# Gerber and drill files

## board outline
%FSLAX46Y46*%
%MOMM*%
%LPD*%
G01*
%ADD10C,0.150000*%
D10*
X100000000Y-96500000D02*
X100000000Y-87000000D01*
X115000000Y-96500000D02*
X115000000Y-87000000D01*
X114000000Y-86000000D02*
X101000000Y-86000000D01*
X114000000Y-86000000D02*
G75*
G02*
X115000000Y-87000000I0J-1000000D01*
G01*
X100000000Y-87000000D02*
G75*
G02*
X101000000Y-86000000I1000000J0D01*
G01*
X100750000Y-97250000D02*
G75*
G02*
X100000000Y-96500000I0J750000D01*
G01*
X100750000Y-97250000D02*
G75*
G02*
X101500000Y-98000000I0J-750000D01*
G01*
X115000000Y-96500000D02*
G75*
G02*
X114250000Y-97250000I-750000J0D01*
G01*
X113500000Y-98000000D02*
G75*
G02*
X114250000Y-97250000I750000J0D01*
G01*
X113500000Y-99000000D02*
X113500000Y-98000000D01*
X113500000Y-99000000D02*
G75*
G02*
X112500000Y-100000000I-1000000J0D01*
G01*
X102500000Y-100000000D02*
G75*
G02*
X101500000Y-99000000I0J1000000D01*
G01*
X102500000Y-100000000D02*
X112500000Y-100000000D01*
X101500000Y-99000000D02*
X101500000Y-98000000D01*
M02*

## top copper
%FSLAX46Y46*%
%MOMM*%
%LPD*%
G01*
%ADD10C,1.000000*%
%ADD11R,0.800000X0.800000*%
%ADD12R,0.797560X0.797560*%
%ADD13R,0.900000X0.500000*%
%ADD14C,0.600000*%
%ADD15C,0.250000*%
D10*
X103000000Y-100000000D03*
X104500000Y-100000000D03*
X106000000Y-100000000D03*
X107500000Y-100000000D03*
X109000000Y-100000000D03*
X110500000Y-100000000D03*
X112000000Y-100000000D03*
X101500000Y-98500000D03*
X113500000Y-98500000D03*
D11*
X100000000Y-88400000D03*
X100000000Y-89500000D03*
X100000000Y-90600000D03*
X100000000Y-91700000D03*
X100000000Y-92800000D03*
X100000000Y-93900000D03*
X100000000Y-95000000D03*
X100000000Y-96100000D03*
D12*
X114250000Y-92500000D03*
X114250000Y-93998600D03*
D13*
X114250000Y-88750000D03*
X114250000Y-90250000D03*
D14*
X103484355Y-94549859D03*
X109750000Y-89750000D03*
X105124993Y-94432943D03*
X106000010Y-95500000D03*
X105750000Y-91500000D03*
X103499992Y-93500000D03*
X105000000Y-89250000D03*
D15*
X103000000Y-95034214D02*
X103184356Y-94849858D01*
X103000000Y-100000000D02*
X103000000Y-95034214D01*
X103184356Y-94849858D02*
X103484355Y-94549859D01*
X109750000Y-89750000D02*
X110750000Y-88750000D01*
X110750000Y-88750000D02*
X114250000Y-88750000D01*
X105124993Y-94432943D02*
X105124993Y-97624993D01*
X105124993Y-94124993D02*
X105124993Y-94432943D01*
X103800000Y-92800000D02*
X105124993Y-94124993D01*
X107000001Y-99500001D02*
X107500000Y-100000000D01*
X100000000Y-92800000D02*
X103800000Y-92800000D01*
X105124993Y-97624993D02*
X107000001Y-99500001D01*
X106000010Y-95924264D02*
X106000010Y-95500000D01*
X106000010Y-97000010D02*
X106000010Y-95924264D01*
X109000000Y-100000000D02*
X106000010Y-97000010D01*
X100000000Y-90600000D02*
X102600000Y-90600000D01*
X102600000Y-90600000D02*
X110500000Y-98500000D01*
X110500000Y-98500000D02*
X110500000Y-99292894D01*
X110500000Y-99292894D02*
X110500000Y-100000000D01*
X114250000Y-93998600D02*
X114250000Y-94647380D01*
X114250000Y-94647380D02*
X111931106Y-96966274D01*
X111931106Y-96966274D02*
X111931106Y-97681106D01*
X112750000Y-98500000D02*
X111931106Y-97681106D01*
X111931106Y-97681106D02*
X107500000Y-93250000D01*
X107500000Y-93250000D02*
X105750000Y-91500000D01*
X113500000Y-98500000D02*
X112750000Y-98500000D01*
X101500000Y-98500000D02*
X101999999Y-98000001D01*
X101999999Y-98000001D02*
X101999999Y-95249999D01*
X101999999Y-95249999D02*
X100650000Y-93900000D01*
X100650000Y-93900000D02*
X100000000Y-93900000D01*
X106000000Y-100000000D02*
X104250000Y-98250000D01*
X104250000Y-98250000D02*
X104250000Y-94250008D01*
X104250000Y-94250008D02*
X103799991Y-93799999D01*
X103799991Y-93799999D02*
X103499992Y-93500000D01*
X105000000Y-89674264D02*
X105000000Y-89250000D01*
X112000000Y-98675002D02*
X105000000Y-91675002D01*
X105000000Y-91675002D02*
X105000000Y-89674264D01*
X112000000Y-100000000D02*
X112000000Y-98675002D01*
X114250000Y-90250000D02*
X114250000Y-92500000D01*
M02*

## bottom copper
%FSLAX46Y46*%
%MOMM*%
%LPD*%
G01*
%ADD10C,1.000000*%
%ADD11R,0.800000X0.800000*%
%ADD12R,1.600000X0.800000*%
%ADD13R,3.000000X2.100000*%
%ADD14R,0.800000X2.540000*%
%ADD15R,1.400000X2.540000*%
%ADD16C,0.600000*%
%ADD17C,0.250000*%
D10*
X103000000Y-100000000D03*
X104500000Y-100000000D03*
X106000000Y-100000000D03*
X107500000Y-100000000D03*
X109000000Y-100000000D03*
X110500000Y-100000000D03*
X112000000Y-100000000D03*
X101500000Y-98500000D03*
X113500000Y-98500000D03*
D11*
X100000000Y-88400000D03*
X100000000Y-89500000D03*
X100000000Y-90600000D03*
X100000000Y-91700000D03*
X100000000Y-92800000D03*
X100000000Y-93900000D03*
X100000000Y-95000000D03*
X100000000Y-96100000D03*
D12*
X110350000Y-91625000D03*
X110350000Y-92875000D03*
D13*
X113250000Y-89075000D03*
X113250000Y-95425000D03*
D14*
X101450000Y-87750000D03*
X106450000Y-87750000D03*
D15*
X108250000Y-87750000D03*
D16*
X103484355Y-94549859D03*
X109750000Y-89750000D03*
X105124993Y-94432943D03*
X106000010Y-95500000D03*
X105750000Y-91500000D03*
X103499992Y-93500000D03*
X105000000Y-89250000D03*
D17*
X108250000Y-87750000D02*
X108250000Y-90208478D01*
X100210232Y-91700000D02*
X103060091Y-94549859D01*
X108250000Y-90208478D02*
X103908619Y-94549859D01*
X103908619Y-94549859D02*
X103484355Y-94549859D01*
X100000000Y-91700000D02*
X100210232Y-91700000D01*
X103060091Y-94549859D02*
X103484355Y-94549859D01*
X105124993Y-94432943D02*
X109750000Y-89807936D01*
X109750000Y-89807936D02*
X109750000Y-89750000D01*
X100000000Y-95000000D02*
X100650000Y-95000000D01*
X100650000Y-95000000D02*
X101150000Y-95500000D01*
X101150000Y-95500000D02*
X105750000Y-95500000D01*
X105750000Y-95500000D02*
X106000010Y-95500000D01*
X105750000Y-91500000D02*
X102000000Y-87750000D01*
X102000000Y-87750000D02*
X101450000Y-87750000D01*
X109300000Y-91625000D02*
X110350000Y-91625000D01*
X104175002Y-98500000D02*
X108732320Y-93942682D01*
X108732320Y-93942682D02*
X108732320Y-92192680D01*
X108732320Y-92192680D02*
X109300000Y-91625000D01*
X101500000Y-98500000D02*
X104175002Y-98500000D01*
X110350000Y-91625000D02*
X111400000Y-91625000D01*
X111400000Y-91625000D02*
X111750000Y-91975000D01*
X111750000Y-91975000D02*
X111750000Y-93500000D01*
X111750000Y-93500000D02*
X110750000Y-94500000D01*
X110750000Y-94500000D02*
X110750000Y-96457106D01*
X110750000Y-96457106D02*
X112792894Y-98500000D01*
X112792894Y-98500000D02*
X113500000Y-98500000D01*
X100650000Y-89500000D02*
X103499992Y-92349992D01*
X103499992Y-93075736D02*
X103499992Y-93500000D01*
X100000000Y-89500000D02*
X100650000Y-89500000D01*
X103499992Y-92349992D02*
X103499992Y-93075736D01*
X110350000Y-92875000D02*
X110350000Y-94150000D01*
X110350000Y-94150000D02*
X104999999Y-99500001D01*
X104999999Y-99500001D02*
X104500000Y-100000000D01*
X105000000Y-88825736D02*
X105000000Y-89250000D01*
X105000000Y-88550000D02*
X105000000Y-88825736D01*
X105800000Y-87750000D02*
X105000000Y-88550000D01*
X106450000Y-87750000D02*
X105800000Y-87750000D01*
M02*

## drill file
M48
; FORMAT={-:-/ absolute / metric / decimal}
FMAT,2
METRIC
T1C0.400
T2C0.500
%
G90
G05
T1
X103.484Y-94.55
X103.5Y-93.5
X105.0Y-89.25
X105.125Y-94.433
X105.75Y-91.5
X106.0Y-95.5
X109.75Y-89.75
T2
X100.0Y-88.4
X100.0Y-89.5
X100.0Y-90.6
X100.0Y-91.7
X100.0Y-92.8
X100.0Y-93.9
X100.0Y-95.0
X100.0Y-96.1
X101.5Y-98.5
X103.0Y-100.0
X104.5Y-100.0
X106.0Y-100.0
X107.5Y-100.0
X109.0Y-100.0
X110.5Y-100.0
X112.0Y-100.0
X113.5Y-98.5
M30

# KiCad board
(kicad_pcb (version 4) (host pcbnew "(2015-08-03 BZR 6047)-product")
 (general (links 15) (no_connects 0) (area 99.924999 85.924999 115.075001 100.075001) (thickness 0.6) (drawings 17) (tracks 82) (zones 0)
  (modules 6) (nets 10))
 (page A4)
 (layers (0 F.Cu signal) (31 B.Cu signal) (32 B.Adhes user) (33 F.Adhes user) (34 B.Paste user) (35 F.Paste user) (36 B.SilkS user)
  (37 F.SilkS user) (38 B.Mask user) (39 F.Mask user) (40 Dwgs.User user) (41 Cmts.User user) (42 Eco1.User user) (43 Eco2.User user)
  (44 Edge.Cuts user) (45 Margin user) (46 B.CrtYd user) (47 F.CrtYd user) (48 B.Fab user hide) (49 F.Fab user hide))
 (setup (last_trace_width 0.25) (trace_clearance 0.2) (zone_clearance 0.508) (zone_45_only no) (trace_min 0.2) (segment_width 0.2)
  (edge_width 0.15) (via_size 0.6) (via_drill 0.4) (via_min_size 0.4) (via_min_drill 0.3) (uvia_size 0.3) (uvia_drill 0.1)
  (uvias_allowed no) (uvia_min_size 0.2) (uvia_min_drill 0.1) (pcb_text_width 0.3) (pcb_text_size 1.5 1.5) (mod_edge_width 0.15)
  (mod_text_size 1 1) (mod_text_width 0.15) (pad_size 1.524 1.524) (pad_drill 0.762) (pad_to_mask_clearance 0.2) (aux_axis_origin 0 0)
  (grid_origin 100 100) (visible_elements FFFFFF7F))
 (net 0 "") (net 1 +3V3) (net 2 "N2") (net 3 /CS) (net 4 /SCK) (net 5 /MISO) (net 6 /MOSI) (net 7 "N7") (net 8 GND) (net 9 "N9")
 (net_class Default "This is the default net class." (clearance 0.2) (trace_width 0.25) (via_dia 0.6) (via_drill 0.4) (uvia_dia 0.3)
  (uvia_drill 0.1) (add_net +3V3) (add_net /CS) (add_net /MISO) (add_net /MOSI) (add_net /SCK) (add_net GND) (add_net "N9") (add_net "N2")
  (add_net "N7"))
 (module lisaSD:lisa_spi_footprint (layer F.Cu) (at 100 100)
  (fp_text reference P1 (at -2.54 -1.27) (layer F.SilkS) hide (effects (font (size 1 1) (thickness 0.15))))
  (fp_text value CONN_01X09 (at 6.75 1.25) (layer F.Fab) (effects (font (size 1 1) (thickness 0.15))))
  (pad 2 thru_hole circle (at 3 0) (size 1 1) (drill 0.5) (layers *.Cu *.Mask F.SilkS) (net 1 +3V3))
  (pad 3 thru_hole circle (at 4.5 0) (size 1 1) (drill 0.5) (layers *.Cu *.Mask F.SilkS) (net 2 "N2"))
  (pad 4 thru_hole circle (at 6 0) (size 1 1) (drill 0.5) (layers *.Cu *.Mask F.SilkS) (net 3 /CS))
  (pad 5 thru_hole circle (at 7.5 0) (size 1 1) (drill 0.5) (layers *.Cu *.Mask F.SilkS) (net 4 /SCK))
  (pad 6 thru_hole circle (at 9 0) (size 1 1) (drill 0.5) (layers *.Cu *.Mask F.SilkS) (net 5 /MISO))
  (pad 7 thru_hole circle (at 10.5 0) (size 1 1) (drill 0.5) (layers *.Cu *.Mask F.SilkS) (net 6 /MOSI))
  (pad 8 thru_hole circle (at 12 0) (size 1 1) (drill 0.5) (layers *.Cu *.Mask F.SilkS) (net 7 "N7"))
  (pad 1 thru_hole circle (at 1.5 -1.5) (size 1 1) (drill 0.5) (layers *.Cu *.Mask F.SilkS) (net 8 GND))
  (pad 9 thru_hole circle (at 13.5 -1.5) (size 1 1) (drill 0.5) (layers *.Cu *.Mask F.SilkS) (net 8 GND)))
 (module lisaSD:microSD (layer F.Cu) (at 100 97.1 90)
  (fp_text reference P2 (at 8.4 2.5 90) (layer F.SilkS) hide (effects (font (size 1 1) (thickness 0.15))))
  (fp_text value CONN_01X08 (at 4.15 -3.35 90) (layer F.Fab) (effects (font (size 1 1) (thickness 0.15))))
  (pad 1 thru_hole rect (at 8.7 0 90) (size 0.8 0.8) (drill 0.5) (layers *.Cu *.Mask F.SilkS))
  (pad 2 thru_hole rect (at 7.6 0 90) (size 0.8 0.8) (drill 0.5) (layers *.Cu *.Mask F.SilkS) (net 3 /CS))
  (pad 3 thru_hole rect (at 6.5 0 90) (size 0.8 0.8) (drill 0.5) (layers *.Cu *.Mask F.SilkS) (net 6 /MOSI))
  (pad 4 thru_hole rect (at 5.4 0 90) (size 0.8 0.8) (drill 0.5) (layers *.Cu *.Mask F.SilkS) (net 1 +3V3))
  (pad 5 thru_hole rect (at 4.3 0 90) (size 0.8 0.8) (drill 0.5) (layers *.Cu *.Mask F.SilkS) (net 4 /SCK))
  (pad 6 thru_hole rect (at 3.2 0 90) (size 0.8 0.8) (drill 0.5) (layers *.Cu *.Mask F.SilkS) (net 8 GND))
  (pad 7 thru_hole rect (at 2.1 0 90) (size 0.8 0.8) (drill 0.5) (layers *.Cu *.Mask F.SilkS) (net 5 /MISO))
  (pad 8 thru_hole rect (at 1 0 90) (size 0.8 0.8) (drill 0.5) (layers *.Cu *.Mask F.SilkS)))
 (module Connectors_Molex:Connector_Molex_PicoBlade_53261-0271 (layer B.Cu) (at 113.25 92.25 270)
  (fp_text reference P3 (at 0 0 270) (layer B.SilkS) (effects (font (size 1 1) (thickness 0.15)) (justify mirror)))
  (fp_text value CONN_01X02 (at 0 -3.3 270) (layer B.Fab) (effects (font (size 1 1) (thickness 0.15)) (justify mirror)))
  (pad 1 smd rect (at -0.625 2.9 270) (size 0.8 1.6) (layers B.Cu B.Paste B.Mask) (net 8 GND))
  (pad 2 smd rect (at 0.625 2.9 270) (size 0.8 1.6) (layers B.Cu B.Paste B.Mask) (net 2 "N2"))
  (pad "" smd rect (at -3.175 0 270) (size 2.1 3) (layers B.Cu B.Paste B.Mask))
  (pad "" smd rect (at 3.175 0 270) (size 2.1 3) (layers B.Cu B.Paste B.Mask)))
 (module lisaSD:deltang (layer B.Cu) (at 100.65 87.85)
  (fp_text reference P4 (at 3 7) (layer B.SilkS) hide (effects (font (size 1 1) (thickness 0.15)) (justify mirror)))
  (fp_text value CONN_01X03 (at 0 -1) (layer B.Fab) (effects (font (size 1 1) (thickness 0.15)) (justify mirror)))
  (pad 1 smd rect (at 0.8 -0.1) (size 0.8 2.54) (layers B.Cu B.Paste B.Mask) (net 8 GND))
  (pad 2 smd rect (at 5.8 -0.1) (size 0.8 2.54) (layers B.Cu B.Paste B.Mask) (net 7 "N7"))
  (pad 3 smd rect (at 7.6 -0.1) (size 1.4 2.54) (layers B.Cu B.Paste B.Mask) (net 1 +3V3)))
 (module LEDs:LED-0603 (layer F.Cu) (at 114.25 93.2493 90)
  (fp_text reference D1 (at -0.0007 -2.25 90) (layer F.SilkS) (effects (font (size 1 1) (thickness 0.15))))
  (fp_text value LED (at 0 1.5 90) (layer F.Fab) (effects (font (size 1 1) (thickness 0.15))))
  (pad 2 smd rect (at 0.7493 0 270) (size 0.79756 0.79756) (layers F.Cu F.Paste F.Mask) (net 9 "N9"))
  (pad 1 smd rect (at -0.7493 0 270) (size 0.79756 0.79756) (layers F.Cu F.Paste F.Mask) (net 8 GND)))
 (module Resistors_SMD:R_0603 (layer F.Cu) (at 114.25 89.5 270)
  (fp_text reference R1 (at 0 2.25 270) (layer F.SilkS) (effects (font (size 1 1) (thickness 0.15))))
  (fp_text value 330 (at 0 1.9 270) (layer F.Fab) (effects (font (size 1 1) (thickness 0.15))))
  (pad 1 smd rect (at -0.75 0 270) (size 0.5 0.9) (layers F.Cu F.Paste F.Mask) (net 4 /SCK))
  (pad 2 smd rect (at 0.75 0 270) (size 0.5 0.9) (layers F.Cu F.Paste F.Mask) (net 9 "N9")))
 (gr_line (start 100 96.5) (end 100 87) (layer Edge.Cuts) (width 0.15))
 (gr_line (start 115 96.5) (end 115 87) (layer Edge.Cuts) (width 0.15))
 (gr_line (start 114 86) (end 101 86) (angle 90) (layer Edge.Cuts) (width 0.15))
 (gr_arc (start 114 87) (end 114 86) (angle 90) (layer Edge.Cuts) (width 0.15))
 (gr_arc (start 101 87) (end 100 87) (angle 90) (layer Edge.Cuts) (width 0.15))
 (gr_arc (start 100.75 96.5) (end 100.75 97.25) (angle 90) (layer Edge.Cuts) (width 0.15))
 (gr_arc (start 100.75 98) (end 100.75 97.25) (angle 90) (layer Edge.Cuts) (width 0.15))
 (gr_arc (start 114.25 96.5) (end 115 96.5) (angle 90) (layer Edge.Cuts) (width 0.15))
 (gr_arc (start 114.25 98) (end 113.5 98) (angle 90) (layer Edge.Cuts) (width 0.15))
 (gr_line (start 113.5 99) (end 113.5 98) (angle 90) (layer Edge.Cuts) (width 0.15))
 (gr_arc (start 112.5 99) (end 113.5 99) (angle 90) (layer Edge.Cuts) (width 0.15))
 (gr_arc (start 102.5 99) (end 102.5 100) (angle 90) (layer Edge.Cuts) (width 0.15))
 (gr_line (start 102.5 100) (end 112.5 100) (angle 90) (layer Edge.Cuts) (width 0.15))
 (gr_line (start 101.5 99) (end 101.5 98) (angle 90) (layer Edge.Cuts) (width 0.15))
 (segment (start 103 95.034214) (end 103.184356 94.849858) (width 0.25) (layer F.Cu) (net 1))
 (segment (start 108.25 87.75) (end 108.25 90.208478) (width 0.25) (layer B.Cu) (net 1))
 (segment (start 100.210232 91.7) (end 103.060091 94.549859) (width 0.25) (layer B.Cu) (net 1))
 (segment (start 108.25 90.208478) (end 103.908619 94.549859) (width 0.25) (layer B.Cu) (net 1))
 (segment (start 103 100) (end 103 95.034214) (width 0.25) (layer F.Cu) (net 1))
 (segment (start 103.908619 94.549859) (end 103.484355 94.549859) (width 0.25) (layer B.Cu) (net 1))
 (via (at 103.484355 94.549859) (size 0.6) (drill 0.4) (layers F.Cu B.Cu) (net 1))
 (segment (start 100 91.7) (end 100.210232 91.7) (width 0.25) (layer B.Cu) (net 1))
 (segment (start 103.060091 94.549859) (end 103.484355 94.549859) (width 0.25) (layer B.Cu) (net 1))
 (segment (start 103.184356 94.849858) (end 103.484355 94.549859) (width 0.25) (layer F.Cu) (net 1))
 (segment (start 109.75 89.75) (end 110.75 88.75) (width 0.25) (layer F.Cu) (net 4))
 (segment (start 110.75 88.75) (end 114.25 88.75) (width 0.25) (layer F.Cu) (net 4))
 (segment (start 105.124993 94.432943) (end 109.75 89.807936) (width 0.25) (layer B.Cu) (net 4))
 (segment (start 109.75 89.807936) (end 109.75 89.75) (width 0.25) (layer B.Cu) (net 4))
 (via (at 109.75 89.75) (size 0.6) (drill 0.4) (layers F.Cu B.Cu) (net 4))
 (segment (start 105.124993 94.432943) (end 105.124993 97.624993) (width 0.25) (layer F.Cu) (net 4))
 (segment (start 105.124993 94.124993) (end 105.124993 94.432943) (width 0.25) (layer F.Cu) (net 4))
 (via (at 105.124993 94.432943) (size 0.6) (drill 0.4) (layers F.Cu B.Cu) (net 4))
 (segment (start 103.8 92.8) (end 105.124993 94.124993) (width 0.25) (layer F.Cu) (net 4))
 (segment (start 107.000001 99.500001) (end 107.5 100) (width 0.25) (layer F.Cu) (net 4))
 (segment (start 100 92.8) (end 103.8 92.8) (width 0.25) (layer F.Cu) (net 4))
 (segment (start 105.124993 97.624993) (end 107.000001 99.500001) (width 0.25) (layer F.Cu) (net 4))
 (segment (start 100 95) (end 100.65 95) (width 0.25) (layer B.Cu) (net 5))
 (segment (start 100.65 95) (end 101.15 95.5) (width 0.25) (layer B.Cu) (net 5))
 (segment (start 101.15 95.5) (end 105.75 95.5) (width 0.25) (layer B.Cu) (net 5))
 (segment (start 105.75 95.5) (end 106.00001 95.5) (width 0.25) (layer B.Cu) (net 5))
 (segment (start 106.00001 95.924264) (end 106.00001 95.5) (width 0.25) (layer F.Cu) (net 5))
 (segment (start 106.00001 97.00001) (end 106.00001 95.924264) (width 0.25) (layer F.Cu) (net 5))
 (via (at 106.00001 95.5) (size 0.6) (drill 0.4) (layers F.Cu B.Cu) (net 5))
 (segment (start 109 100) (end 106.00001 97.00001) (width 0.25) (layer F.Cu) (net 5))
 (segment (start 100 90.6) (end 102.6 90.6) (width 0.25) (layer F.Cu) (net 6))
 (segment (start 102.6 90.6) (end 110.5 98.5) (width 0.25) (layer F.Cu) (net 6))
 (segment (start 110.5 98.5) (end 110.5 99.292894) (width 0.25) (layer F.Cu) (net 6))
 (segment (start 110.5 99.292894) (end 110.5 100) (width 0.25) (layer F.Cu) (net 6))
 (segment (start 114.25 93.9986) (end 114.25 94.64738) (width 0.25) (layer F.Cu) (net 8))
 (segment (start 114.25 94.64738) (end 111.931106 96.966274) (width 0.25) (layer F.Cu) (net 8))
 (segment (start 111.931106 96.966274) (end 111.931106 97.681106) (width 0.25) (layer F.Cu) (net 8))
 (segment (start 112.75 98.5) (end 111.931106 97.681106) (width 0.25) (layer F.Cu) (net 8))
 (segment (start 111.931106 97.681106) (end 107.5 93.25) (width 0.25) (layer F.Cu) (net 8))
 (segment (start 105.75 91.5) (end 102 87.75) (width 0.25) (layer B.Cu) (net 8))
 (segment (start 102 87.75) (end 101.45 87.75) (width 0.25) (layer B.Cu) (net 8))
 (segment (start 107.5 93.25) (end 105.75 91.5) (width 0.25) (layer F.Cu) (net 8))
 (via (at 105.75 91.5) (size 0.6) (drill 0.4) (layers F.Cu B.Cu) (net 8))
 (segment (start 113.5 98.5) (end 112.75 98.5) (width 0.25) (layer F.Cu) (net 8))
 (segment (start 109.3 91.625) (end 110.35 91.625) (width 0.25) (layer B.Cu) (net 8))
 (segment (start 104.175002 98.5) (end 108.73232 93.942682) (width 0.25) (layer B.Cu) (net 8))
 (segment (start 108.73232 93.942682) (end 108.73232 92.19268) (width 0.25) (layer B.Cu) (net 8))
 (segment (start 108.73232 92.19268) (end 109.3 91.625) (width 0.25) (layer B.Cu) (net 8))
 (segment (start 101.5 98.5) (end 104.175002 98.5) (width 0.25) (layer B.Cu) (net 8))
 (segment (start 110.35 91.625) (end 111.4 91.625) (width 0.25) (layer B.Cu) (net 8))
 (segment (start 111.4 91.625) (end 111.75 91.975) (width 0.25) (layer B.Cu) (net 8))
 (segment (start 111.75 91.975) (end 111.75 93.5) (width 0.25) (layer B.Cu) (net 8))
 (segment (start 111.75 93.5) (end 110.75 94.5) (width 0.25) (layer B.Cu) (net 8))
 (segment (start 110.75 94.5) (end 110.75 96.457106) (width 0.25) (layer B.Cu) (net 8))
 (segment (start 110.75 96.457106) (end 112.792894 98.5) (width 0.25) (layer B.Cu) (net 8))
 (segment (start 112.792894 98.5) (end 113.5 98.5) (width 0.25) (layer B.Cu) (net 8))
 (segment (start 101.5 98.5) (end 101.999999 98.000001) (width 0.25) (layer F.Cu) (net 8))
 (segment (start 101.999999 98.000001) (end 101.999999 95.249999) (width 0.25) (layer F.Cu) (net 8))
 (segment (start 101.999999 95.249999) (end 100.65 93.9) (width 0.25) (layer F.Cu) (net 8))
 (segment (start 100.65 93.9) (end 100 93.9) (width 0.25) (layer F.Cu) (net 8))
 (segment (start 100.65 89.5) (end 103.499992 92.349992) (width 0.25) (layer B.Cu) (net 3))
 (segment (start 103.499992 93.075736) (end 103.499992 93.5) (width 0.25) (layer B.Cu) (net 3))
 (segment (start 106 100) (end 104.25 98.25) (width 0.25) (layer F.Cu) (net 3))
 (segment (start 100 89.5) (end 100.65 89.5) (width 0.25) (layer B.Cu) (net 3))
 (segment (start 104.25 98.25) (end 104.25 94.250008) (width 0.25) (layer F.Cu) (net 3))
 (via (at 103.499992 93.5) (size 0.6) (drill 0.4) (layers F.Cu B.Cu) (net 3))
 (segment (start 103.499992 92.349992) (end 103.499992 93.075736) (width 0.25) (layer B.Cu) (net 3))
 (segment (start 104.25 94.250008) (end 103.799991 93.799999) (width 0.25) (layer F.Cu) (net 3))
 (segment (start 103.799991 93.799999) (end 103.499992 93.5) (width 0.25) (layer F.Cu) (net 3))
 (segment (start 110.35 92.875) (end 110.35 94.15) (width 0.25) (layer B.Cu) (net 2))
 (segment (start 110.35 94.15) (end 104.999999 99.500001) (width 0.25) (layer B.Cu) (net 2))
 (segment (start 104.999999 99.500001) (end 104.5 100) (width 0.25) (layer B.Cu) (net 2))
 (segment (start 105 89.674264) (end 105 89.25) (width 0.25) (layer F.Cu) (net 7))
 (segment (start 112 98.675002) (end 105 91.675002) (width 0.25) (layer F.Cu) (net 7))
 (segment (start 105 91.675002) (end 105 89.674264) (width 0.25) (layer F.Cu) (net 7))
 (segment (start 112 100) (end 112 98.675002) (width 0.25) (layer F.Cu) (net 7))
 (segment (start 105 88.825736) (end 105 89.25) (width 0.25) (layer B.Cu) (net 7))
 (segment (start 105 88.55) (end 105 88.825736) (width 0.25) (layer B.Cu) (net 7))
 (segment (start 105.8 87.75) (end 105 88.55) (width 0.25) (layer B.Cu) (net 7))
 (segment (start 106.45 87.75) (end 105.8 87.75) (width 0.25) (layer B.Cu) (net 7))
 (via (at 105 89.25) (size 0.6) (drill 0.4) (layers F.Cu B.Cu) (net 7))
 (segment (start 114.25 90.25) (end 114.25 92.5) (width 0.25) (layer F.Cu) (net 9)))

